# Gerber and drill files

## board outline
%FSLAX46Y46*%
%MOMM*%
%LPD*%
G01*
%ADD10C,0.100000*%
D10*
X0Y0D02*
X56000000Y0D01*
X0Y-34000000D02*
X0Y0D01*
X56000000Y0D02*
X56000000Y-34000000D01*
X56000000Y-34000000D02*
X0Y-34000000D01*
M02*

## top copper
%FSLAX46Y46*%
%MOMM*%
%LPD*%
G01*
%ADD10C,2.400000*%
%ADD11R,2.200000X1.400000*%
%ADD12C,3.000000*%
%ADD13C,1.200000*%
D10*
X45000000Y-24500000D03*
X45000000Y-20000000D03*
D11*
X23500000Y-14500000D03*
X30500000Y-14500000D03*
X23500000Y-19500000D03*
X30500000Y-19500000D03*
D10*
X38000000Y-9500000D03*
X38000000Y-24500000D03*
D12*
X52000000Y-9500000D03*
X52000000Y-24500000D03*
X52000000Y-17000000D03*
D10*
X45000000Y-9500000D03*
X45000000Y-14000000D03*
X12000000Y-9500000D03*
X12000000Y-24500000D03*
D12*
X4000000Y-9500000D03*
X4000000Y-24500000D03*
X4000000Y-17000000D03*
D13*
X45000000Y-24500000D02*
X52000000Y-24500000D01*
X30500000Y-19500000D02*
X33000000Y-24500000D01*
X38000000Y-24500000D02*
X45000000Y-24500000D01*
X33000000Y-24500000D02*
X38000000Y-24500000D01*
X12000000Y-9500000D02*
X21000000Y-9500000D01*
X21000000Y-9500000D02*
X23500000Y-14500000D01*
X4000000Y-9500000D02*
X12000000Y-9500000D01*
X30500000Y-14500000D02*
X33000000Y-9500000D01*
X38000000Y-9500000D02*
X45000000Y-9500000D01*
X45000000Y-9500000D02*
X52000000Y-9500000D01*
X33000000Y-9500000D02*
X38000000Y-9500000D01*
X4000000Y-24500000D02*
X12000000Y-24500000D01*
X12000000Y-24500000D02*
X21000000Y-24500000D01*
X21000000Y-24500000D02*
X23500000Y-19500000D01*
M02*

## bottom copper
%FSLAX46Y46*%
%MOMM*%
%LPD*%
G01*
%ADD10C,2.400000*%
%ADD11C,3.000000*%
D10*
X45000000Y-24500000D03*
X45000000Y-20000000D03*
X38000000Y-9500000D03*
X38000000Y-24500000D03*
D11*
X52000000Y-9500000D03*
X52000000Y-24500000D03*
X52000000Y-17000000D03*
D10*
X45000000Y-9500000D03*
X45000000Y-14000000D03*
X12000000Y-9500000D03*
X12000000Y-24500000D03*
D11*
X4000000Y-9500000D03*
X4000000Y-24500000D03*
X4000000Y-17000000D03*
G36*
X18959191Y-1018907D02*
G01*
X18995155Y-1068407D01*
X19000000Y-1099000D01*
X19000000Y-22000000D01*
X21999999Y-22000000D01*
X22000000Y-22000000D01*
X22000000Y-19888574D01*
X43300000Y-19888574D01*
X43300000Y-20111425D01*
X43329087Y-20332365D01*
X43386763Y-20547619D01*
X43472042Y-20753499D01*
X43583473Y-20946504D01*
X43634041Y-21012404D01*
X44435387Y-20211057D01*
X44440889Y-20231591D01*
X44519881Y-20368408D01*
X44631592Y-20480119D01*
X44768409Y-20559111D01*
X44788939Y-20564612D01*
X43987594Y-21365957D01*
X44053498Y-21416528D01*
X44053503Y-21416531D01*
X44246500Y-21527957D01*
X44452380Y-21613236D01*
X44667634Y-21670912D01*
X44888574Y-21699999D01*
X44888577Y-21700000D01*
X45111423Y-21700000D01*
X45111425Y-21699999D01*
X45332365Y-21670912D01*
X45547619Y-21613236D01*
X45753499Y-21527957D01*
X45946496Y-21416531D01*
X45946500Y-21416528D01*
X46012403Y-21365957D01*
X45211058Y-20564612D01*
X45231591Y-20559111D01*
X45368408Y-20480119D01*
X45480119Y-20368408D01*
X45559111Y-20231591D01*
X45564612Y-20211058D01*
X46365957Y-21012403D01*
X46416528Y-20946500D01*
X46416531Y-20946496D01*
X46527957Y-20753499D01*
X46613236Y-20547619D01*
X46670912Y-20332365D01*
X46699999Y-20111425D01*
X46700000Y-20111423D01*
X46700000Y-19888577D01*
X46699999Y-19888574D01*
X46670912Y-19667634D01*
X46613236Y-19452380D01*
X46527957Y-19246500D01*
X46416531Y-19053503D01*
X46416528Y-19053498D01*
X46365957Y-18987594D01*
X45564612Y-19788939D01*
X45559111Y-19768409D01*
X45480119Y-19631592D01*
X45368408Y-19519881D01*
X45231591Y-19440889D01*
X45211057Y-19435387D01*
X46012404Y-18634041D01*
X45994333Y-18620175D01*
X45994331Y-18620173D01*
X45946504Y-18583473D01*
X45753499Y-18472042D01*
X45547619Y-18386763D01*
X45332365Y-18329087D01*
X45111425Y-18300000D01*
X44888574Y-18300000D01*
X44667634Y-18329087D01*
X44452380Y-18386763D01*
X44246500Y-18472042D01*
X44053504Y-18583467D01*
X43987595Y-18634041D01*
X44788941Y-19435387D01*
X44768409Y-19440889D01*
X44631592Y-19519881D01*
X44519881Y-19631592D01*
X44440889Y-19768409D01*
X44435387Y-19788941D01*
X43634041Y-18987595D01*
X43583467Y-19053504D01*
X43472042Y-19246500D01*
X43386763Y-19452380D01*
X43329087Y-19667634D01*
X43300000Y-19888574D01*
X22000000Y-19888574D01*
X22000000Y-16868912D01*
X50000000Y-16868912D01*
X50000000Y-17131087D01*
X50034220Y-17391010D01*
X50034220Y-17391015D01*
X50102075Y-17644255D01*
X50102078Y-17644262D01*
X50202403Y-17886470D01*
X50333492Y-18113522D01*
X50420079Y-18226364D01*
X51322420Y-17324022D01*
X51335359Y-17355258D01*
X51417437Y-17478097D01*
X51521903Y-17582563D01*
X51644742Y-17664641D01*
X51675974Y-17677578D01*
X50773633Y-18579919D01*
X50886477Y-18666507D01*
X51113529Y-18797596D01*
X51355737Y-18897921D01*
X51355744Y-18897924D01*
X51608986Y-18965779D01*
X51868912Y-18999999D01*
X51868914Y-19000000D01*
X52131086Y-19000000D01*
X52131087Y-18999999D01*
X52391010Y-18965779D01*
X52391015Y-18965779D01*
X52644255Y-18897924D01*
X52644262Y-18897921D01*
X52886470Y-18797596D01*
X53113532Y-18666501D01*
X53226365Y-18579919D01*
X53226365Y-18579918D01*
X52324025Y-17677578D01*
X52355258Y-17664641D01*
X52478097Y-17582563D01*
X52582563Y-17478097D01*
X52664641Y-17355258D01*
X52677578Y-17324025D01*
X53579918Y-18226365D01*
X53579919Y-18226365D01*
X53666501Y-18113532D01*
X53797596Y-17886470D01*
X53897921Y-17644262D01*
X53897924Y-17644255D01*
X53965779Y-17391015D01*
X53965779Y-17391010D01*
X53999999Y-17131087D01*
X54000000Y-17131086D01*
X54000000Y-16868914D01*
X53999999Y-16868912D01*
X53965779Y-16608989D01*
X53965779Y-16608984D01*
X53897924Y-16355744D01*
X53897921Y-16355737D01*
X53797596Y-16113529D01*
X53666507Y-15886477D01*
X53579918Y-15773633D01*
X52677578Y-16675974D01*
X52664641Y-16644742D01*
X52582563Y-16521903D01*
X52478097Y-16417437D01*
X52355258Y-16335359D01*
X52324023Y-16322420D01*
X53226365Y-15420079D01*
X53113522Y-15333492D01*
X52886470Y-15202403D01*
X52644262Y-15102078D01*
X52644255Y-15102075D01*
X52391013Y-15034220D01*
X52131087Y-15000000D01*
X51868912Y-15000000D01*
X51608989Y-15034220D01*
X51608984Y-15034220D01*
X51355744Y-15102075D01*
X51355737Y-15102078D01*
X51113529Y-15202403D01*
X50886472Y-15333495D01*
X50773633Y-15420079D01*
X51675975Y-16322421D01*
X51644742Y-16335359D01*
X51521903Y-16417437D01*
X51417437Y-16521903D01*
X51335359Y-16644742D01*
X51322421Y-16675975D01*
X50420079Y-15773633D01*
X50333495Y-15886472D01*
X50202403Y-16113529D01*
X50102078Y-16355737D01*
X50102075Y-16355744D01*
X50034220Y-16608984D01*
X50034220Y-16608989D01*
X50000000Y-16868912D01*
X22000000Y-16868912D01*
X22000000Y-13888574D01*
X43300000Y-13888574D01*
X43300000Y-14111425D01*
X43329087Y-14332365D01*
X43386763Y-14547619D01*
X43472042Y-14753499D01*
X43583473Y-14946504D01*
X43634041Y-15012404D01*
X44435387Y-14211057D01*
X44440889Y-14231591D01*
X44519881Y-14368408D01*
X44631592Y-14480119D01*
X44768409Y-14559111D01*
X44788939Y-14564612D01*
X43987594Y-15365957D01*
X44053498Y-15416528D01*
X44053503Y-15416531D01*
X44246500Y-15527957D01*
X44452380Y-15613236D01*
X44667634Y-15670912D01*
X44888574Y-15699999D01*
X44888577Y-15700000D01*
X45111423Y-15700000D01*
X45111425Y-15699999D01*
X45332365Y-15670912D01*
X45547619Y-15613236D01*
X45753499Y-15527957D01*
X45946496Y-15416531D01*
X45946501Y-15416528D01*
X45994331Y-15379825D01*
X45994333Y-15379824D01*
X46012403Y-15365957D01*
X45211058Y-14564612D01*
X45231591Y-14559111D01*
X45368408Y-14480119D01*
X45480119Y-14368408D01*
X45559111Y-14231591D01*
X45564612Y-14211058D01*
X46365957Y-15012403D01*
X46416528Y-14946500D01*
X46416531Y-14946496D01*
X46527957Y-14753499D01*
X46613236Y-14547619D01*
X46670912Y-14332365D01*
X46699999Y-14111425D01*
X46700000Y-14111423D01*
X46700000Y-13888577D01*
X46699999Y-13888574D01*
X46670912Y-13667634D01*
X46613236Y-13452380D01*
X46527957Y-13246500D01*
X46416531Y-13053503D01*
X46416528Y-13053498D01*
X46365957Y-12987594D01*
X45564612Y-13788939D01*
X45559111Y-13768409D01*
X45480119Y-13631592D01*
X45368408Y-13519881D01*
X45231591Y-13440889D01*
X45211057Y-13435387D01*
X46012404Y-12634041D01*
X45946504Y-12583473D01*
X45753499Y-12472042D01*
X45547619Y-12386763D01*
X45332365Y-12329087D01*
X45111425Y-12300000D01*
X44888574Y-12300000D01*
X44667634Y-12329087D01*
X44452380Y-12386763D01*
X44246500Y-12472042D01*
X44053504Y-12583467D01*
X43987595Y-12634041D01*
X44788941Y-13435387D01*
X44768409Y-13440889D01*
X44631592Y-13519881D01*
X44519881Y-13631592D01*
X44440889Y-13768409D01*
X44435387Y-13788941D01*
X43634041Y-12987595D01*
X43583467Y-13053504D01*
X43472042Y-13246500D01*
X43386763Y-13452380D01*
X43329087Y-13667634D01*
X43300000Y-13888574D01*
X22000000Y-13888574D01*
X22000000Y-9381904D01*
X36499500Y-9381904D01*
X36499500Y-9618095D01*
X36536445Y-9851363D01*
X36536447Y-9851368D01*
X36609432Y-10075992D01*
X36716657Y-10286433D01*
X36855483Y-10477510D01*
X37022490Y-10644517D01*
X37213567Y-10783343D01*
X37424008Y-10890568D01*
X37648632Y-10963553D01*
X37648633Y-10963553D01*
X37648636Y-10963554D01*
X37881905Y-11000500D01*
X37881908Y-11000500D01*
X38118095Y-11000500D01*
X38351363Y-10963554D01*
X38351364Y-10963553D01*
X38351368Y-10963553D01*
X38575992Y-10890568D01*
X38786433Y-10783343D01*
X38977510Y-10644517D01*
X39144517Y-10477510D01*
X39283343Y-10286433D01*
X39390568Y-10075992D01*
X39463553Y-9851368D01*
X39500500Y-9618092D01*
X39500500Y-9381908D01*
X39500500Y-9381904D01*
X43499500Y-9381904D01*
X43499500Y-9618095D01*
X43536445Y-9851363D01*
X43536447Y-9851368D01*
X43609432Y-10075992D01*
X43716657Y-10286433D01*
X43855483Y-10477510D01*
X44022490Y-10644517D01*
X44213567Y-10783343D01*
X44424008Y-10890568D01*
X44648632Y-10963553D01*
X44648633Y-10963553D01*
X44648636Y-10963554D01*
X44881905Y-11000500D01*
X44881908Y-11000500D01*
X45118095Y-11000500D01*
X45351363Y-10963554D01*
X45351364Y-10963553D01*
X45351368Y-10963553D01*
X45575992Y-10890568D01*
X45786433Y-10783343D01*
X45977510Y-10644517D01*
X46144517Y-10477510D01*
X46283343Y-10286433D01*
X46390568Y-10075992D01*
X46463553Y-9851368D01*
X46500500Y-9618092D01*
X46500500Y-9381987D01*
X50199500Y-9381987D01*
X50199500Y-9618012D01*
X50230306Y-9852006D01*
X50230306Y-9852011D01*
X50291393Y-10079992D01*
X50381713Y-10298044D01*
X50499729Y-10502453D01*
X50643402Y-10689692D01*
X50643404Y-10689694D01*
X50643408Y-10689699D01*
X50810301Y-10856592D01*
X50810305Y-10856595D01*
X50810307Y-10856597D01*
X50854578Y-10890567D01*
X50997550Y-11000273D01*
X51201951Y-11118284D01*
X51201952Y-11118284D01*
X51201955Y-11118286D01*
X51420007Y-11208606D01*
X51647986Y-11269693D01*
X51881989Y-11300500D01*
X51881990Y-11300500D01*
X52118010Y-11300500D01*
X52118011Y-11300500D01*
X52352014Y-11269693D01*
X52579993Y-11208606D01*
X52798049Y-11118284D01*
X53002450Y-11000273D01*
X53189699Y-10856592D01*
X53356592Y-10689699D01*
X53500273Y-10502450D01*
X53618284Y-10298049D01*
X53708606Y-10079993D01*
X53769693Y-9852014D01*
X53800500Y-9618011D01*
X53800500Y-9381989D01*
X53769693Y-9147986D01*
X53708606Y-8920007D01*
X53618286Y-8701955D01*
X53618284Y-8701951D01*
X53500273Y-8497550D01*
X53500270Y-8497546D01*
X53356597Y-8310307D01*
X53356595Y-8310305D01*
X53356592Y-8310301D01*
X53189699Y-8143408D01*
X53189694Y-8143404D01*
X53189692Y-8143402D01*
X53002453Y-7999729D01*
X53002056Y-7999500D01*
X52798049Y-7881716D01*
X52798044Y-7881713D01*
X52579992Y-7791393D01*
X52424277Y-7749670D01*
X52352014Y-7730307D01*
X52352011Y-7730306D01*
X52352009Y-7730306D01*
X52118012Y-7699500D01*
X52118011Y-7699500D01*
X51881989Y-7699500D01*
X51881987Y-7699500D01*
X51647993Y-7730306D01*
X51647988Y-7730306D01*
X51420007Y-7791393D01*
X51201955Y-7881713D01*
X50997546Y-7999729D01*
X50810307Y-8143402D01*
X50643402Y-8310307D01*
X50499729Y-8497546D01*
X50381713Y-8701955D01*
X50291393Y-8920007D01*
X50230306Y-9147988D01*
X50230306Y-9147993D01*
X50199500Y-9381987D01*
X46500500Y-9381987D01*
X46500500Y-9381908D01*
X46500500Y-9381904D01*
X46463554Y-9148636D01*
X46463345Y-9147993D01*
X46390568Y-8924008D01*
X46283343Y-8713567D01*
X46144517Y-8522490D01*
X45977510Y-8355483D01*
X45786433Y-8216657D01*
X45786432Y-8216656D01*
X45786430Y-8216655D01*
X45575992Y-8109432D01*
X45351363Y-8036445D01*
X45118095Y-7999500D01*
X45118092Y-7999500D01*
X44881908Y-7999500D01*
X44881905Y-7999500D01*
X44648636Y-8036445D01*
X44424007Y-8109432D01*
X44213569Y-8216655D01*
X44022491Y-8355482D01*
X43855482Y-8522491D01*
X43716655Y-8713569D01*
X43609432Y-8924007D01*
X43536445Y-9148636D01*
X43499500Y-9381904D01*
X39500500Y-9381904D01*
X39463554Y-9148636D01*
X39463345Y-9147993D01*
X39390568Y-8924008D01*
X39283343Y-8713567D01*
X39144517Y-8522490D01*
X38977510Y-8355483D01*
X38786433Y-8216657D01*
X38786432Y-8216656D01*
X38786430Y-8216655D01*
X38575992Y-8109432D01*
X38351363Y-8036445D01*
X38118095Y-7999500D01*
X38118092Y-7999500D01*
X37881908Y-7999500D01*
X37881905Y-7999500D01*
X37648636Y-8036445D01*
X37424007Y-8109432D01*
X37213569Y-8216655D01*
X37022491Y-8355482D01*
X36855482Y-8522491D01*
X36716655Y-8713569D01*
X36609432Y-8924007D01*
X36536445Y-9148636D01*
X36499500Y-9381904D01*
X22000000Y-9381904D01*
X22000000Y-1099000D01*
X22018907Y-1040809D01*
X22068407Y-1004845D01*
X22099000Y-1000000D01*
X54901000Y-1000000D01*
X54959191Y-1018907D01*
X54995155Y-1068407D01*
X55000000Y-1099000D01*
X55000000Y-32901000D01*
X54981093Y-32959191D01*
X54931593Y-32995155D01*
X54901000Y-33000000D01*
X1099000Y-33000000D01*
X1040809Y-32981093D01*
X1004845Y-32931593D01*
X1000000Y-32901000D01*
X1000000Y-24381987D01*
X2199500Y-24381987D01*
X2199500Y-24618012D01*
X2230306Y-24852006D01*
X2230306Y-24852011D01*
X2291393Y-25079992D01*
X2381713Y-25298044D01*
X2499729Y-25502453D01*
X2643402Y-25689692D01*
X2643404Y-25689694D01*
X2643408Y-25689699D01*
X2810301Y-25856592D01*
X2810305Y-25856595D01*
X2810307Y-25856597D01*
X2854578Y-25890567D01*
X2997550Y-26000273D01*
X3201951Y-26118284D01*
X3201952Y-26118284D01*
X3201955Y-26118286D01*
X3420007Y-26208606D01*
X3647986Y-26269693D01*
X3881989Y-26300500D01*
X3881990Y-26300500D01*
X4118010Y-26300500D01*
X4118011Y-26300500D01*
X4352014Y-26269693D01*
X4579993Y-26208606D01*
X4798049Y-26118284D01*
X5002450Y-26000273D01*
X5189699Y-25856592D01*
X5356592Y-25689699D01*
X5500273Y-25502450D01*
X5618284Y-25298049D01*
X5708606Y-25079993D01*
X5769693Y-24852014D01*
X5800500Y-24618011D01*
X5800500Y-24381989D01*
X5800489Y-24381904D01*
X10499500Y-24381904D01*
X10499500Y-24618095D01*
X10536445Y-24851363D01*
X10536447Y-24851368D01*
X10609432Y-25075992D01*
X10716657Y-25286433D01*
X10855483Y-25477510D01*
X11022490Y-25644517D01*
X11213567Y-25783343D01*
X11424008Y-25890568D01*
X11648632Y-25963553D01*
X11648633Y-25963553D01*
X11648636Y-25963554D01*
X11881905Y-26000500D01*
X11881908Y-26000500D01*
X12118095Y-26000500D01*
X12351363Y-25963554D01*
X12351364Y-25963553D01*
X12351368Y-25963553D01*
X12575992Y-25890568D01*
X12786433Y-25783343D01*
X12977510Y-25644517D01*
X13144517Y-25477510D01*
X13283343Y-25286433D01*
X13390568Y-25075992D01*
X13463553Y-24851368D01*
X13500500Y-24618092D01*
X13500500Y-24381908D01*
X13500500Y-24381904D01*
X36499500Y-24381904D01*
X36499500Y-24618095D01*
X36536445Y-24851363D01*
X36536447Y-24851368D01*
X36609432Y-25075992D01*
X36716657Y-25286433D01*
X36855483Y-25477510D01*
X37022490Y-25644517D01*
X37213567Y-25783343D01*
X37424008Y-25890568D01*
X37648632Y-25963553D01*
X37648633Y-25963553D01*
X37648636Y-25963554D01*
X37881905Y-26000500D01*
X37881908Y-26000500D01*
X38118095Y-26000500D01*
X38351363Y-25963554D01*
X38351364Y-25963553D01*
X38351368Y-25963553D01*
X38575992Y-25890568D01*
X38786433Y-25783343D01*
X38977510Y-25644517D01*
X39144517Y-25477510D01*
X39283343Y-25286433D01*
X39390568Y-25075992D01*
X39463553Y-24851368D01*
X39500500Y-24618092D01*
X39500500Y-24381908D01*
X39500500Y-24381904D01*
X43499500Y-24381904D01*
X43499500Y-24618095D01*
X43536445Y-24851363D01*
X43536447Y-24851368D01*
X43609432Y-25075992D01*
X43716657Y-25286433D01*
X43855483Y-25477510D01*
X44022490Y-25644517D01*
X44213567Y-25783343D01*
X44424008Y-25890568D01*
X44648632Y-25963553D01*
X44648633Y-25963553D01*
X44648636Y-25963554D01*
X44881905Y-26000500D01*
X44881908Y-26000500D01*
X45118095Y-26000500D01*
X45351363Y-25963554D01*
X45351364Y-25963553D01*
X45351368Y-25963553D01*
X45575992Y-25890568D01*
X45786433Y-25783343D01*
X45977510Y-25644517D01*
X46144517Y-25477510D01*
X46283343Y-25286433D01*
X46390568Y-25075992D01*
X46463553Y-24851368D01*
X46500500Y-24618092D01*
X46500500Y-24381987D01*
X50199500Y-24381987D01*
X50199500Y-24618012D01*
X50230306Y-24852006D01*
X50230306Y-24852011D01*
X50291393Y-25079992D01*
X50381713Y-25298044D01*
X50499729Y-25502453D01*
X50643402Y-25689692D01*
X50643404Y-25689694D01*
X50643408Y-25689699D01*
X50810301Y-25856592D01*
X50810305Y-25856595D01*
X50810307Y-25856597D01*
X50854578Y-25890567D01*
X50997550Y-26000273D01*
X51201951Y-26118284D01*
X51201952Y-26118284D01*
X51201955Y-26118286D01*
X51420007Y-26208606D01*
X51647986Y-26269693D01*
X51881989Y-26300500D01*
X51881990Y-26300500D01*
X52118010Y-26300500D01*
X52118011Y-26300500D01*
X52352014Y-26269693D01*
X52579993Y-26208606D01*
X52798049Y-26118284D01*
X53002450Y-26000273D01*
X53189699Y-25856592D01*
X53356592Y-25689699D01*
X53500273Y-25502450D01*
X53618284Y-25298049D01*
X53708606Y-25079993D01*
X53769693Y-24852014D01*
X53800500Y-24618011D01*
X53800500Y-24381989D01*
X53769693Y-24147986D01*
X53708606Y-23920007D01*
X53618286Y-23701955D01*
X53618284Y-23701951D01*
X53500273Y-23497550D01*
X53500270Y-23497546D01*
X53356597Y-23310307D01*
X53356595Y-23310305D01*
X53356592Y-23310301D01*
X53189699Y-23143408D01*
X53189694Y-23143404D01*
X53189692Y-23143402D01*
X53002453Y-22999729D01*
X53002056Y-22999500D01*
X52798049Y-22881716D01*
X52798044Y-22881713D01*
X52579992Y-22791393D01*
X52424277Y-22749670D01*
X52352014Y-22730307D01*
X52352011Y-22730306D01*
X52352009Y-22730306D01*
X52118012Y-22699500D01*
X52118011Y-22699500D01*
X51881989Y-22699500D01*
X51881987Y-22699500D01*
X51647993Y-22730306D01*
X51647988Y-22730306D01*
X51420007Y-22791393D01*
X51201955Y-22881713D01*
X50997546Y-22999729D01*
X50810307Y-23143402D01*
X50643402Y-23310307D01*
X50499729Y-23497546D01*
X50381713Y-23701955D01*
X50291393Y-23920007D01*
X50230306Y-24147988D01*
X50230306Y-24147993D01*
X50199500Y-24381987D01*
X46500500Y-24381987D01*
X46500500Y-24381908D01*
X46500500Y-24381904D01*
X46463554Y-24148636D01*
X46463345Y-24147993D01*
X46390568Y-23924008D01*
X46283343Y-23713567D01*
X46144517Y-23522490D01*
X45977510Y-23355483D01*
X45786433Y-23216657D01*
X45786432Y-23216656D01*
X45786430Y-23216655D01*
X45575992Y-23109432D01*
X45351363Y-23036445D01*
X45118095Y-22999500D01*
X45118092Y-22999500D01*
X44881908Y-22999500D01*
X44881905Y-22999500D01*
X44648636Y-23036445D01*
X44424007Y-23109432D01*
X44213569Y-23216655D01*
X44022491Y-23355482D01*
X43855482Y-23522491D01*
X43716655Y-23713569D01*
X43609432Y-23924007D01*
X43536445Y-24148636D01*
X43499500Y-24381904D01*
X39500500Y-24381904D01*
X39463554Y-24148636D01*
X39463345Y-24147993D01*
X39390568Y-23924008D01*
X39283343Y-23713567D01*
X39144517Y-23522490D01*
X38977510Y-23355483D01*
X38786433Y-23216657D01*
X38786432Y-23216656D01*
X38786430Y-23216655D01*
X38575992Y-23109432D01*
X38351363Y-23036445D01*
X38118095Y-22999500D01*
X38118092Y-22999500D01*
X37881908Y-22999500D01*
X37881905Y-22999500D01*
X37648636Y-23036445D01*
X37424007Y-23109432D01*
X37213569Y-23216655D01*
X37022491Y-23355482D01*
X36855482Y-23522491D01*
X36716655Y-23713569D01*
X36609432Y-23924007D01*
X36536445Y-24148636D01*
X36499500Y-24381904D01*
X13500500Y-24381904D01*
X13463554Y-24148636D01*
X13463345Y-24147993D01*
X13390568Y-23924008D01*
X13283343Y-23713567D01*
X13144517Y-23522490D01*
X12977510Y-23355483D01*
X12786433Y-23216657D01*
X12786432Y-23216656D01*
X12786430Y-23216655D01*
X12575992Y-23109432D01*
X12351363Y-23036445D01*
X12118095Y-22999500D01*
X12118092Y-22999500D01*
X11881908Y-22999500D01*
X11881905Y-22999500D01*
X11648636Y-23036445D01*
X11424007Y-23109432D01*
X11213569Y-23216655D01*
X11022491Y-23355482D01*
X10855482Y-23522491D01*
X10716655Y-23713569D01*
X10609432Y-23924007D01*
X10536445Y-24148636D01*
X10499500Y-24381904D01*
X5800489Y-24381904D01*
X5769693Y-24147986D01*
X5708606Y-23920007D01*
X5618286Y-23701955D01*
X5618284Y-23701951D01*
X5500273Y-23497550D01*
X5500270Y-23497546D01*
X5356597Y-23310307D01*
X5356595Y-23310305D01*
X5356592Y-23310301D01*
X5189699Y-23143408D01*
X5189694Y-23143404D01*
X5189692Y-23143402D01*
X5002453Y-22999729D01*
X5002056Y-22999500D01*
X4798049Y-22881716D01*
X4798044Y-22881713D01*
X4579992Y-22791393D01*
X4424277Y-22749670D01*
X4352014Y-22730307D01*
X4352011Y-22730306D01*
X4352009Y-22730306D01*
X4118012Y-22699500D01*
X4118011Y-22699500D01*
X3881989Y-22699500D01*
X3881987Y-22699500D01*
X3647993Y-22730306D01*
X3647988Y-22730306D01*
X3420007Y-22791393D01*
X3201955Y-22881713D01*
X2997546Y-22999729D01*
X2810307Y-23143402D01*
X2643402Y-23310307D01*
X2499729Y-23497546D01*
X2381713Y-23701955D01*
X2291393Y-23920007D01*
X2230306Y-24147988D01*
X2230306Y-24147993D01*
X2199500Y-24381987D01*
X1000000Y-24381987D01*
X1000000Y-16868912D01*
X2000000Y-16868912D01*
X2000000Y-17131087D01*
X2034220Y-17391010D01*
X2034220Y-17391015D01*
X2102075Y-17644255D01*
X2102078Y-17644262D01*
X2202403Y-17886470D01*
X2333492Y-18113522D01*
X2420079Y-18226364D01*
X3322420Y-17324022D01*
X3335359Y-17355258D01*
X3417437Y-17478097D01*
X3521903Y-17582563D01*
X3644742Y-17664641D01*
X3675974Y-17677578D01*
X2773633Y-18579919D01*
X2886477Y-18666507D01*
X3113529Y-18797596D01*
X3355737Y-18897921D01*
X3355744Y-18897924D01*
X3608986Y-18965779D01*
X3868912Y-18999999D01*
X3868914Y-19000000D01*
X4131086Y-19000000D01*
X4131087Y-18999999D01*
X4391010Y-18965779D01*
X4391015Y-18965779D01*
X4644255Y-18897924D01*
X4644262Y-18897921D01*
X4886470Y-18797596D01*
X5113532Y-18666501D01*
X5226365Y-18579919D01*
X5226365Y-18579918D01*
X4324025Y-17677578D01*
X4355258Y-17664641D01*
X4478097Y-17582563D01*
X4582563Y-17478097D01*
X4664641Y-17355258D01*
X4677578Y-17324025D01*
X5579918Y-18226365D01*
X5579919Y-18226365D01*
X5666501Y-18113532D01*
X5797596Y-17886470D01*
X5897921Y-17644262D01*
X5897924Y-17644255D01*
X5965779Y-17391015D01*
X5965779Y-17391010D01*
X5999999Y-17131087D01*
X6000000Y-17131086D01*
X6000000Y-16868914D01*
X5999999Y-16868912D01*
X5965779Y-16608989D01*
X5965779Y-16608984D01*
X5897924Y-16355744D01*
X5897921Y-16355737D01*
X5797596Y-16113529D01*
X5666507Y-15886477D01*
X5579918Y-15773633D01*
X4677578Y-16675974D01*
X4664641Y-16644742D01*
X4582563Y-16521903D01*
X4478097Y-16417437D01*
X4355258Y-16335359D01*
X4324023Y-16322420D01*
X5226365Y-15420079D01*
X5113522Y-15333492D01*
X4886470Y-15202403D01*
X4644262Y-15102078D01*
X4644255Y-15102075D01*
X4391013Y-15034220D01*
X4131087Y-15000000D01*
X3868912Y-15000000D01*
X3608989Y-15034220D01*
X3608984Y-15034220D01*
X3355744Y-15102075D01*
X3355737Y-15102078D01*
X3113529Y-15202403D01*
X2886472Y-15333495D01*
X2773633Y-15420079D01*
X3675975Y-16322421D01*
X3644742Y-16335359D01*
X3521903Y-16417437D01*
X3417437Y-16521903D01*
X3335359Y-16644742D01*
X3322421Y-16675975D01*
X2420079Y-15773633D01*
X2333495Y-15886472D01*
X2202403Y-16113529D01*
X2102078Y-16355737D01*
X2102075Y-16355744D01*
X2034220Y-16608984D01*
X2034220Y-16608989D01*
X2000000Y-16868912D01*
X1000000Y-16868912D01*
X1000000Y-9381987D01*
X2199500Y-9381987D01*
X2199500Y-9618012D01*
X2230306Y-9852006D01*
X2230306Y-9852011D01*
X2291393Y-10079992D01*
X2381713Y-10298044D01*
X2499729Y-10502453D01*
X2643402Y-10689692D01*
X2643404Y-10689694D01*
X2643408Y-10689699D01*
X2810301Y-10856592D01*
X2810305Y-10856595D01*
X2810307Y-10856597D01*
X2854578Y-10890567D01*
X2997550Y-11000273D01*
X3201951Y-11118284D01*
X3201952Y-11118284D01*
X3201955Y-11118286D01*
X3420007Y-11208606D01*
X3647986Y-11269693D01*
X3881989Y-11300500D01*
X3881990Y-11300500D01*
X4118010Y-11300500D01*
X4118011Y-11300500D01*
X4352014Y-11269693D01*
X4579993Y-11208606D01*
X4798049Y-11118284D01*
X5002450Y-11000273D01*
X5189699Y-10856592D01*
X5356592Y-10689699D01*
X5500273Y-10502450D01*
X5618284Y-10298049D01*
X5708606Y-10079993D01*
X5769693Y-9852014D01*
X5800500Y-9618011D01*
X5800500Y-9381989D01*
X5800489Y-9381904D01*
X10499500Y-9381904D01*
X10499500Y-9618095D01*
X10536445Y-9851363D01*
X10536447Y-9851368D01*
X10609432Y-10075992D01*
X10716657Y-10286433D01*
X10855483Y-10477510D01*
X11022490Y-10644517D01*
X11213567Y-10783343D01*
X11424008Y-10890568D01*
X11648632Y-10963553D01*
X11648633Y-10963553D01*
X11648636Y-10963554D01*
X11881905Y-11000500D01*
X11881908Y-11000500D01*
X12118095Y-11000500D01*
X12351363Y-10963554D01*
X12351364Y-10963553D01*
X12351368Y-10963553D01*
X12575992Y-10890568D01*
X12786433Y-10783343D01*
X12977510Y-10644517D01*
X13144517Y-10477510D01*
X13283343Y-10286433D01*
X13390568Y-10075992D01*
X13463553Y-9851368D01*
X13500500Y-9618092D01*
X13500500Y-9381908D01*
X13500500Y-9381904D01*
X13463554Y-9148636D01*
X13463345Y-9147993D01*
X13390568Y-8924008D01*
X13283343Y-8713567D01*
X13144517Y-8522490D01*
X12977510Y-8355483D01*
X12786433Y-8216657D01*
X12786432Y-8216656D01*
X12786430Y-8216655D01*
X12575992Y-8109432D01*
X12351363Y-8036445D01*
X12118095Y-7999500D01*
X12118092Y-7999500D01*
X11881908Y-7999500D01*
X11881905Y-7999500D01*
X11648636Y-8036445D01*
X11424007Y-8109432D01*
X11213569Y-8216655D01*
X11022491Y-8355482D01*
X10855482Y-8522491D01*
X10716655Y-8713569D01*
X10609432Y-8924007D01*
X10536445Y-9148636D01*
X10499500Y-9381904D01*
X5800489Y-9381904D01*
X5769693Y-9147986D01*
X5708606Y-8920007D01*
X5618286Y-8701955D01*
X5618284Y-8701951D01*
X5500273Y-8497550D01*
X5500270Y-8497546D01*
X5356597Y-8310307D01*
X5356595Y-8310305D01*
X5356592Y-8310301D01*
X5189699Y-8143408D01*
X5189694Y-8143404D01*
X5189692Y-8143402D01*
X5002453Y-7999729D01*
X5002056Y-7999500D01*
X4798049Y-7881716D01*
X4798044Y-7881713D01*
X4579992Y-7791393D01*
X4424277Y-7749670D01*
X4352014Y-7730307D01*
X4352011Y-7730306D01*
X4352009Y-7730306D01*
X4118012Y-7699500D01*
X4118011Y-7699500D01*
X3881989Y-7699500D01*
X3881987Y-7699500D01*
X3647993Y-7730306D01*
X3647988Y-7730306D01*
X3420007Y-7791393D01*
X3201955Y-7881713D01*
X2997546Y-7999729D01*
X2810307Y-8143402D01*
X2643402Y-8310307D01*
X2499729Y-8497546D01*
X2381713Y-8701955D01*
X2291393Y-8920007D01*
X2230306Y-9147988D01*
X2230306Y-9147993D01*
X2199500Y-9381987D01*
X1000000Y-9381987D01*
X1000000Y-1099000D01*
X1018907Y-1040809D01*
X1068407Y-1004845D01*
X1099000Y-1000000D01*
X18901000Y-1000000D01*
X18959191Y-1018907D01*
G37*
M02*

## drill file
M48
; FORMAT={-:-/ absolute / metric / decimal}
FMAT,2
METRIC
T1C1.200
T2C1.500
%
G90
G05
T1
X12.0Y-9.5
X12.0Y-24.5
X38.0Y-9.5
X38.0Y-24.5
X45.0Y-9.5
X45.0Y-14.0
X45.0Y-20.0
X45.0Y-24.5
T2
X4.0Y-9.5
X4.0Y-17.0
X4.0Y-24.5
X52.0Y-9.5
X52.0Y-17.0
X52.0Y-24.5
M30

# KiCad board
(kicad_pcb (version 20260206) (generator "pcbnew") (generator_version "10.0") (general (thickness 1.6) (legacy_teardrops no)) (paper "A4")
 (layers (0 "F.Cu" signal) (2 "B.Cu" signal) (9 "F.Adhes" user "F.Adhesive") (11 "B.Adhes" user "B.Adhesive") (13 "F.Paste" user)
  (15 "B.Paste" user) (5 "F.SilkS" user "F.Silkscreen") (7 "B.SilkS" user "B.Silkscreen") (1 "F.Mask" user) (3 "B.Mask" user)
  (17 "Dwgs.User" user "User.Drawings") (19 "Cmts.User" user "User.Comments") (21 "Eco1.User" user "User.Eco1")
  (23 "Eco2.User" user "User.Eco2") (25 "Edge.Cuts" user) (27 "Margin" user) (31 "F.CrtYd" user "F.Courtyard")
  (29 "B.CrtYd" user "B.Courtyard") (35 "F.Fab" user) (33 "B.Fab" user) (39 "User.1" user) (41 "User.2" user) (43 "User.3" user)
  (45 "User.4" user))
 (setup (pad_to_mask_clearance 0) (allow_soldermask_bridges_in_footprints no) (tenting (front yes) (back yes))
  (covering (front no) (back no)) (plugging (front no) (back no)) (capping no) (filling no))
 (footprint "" (layer "F.Cu") (at 0 0)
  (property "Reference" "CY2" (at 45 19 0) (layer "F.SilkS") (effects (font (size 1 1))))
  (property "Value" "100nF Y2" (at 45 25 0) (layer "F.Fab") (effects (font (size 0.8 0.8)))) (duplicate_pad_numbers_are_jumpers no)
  (pad "1" thru_hole circle (at 45 24.5) (size 2.4 2.4) (drill 1.2) (layers "*.Cu" "*.Mask") (remove_unused_layers no) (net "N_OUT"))
  (pad "2" thru_hole circle (at 45 20) (size 2.4 2.4) (drill 1.2) (layers "*.Cu" "*.Mask") (remove_unused_layers no) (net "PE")))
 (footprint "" (layer "F.Cu") (at 0 0)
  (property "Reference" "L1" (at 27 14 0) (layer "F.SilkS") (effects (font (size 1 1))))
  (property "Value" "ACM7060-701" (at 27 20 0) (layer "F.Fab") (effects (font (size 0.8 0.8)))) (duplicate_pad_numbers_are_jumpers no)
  (pad "1" smd rect (at 23.5 14.5) (size 2.2 1.4) (layers "F.Cu" "F.Mask" "F.Paste") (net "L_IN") (thermal_bridge_angle 45))
  (pad "2" smd rect (at 30.5 14.5) (size 2.2 1.4) (layers "F.Cu" "F.Mask" "F.Paste") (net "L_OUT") (thermal_bridge_angle 45))
  (pad "3" smd rect (at 23.5 19.5) (size 2.2 1.4) (layers "F.Cu" "F.Mask" "F.Paste") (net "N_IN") (thermal_bridge_angle 45))
  (pad "4" smd rect (at 30.5 19.5) (size 2.2 1.4) (layers "F.Cu" "F.Mask" "F.Paste") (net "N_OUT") (thermal_bridge_angle 45)))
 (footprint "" (layer "F.Cu") (at 0 0)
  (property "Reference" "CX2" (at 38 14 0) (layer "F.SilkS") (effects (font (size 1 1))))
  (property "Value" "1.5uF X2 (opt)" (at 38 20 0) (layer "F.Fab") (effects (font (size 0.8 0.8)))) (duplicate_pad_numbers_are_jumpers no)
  (pad "1" thru_hole circle (at 38 9.5) (size 2.4 2.4) (drill 1.2) (layers "*.Cu" "*.Mask") (remove_unused_layers no) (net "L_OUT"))
  (pad "2" thru_hole circle (at 38 24.5) (size 2.4 2.4) (drill 1.2) (layers "*.Cu" "*.Mask") (remove_unused_layers no) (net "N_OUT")))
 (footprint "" (layer "F.Cu") (at 0 0)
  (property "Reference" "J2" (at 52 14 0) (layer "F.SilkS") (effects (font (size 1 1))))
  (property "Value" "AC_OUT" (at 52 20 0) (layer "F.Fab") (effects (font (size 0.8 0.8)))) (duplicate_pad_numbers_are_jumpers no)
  (pad "1" thru_hole circle (at 52 9.5) (size 3 3) (drill 1.5) (layers "*.Cu" "*.Mask") (remove_unused_layers no) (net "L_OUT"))
  (pad "2" thru_hole circle (at 52 24.5) (size 3 3) (drill 1.5) (layers "*.Cu" "*.Mask") (remove_unused_layers no) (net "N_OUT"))
  (pad "3" thru_hole circle (at 52 17) (size 3 3) (drill 1.5) (layers "*.Cu" "*.Mask") (remove_unused_layers no) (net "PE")))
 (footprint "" (layer "F.Cu") (at 0 0)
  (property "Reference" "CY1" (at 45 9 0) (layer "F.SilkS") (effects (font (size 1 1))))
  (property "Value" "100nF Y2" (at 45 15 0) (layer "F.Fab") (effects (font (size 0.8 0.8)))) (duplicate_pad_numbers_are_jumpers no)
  (pad "1" thru_hole circle (at 45 9.5) (size 2.4 2.4) (drill 1.2) (layers "*.Cu" "*.Mask") (remove_unused_layers no) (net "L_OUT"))
  (pad "2" thru_hole circle (at 45 14) (size 2.4 2.4) (drill 1.2) (layers "*.Cu" "*.Mask") (remove_unused_layers no) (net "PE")))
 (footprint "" (layer "F.Cu") (at 0 0)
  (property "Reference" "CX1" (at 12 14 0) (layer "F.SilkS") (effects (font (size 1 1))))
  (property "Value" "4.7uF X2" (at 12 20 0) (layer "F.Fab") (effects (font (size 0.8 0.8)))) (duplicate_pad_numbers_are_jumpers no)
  (pad "1" thru_hole circle (at 12 9.5) (size 2.4 2.4) (drill 1.2) (layers "*.Cu" "*.Mask") (remove_unused_layers no) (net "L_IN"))
  (pad "2" thru_hole circle (at 12 24.5) (size 2.4 2.4) (drill 1.2) (layers "*.Cu" "*.Mask") (remove_unused_layers no) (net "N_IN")))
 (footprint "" (layer "F.Cu") (at 0 0)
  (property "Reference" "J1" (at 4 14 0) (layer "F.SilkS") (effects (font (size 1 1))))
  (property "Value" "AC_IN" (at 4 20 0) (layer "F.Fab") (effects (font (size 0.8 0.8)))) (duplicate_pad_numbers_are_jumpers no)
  (pad "1" thru_hole circle (at 4 9.5) (size 3 3) (drill 1.5) (layers "*.Cu" "*.Mask") (remove_unused_layers no) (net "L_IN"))
  (pad "2" thru_hole circle (at 4 24.5) (size 3 3) (drill 1.5) (layers "*.Cu" "*.Mask") (remove_unused_layers no) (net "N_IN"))
  (pad "3" thru_hole circle (at 4 17) (size 3 3) (drill 1.5) (layers "*.Cu" "*.Mask") (remove_unused_layers no) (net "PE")))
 (gr_line (start 0 0) (end 56 0) (stroke (width 0.1) (type default)) (layer "Edge.Cuts"))
 (gr_line (start 0 34) (end 0 0) (stroke (width 0.1) (type default)) (layer "Edge.Cuts"))
 (gr_line (start 56 0) (end 56 34) (stroke (width 0.1) (type default)) (layer "Edge.Cuts"))
 (gr_line (start 56 34) (end 0 34) (stroke (width 0.1) (type default)) (layer "Edge.Cuts"))
 (segment (start 45 24.5) (end 52 24.5) (width 1.2) (layer "F.Cu") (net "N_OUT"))
 (segment (start 30.5 19.5) (end 33 24.5) (width 1.2) (layer "F.Cu") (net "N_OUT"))
 (segment (start 38 24.5) (end 45 24.5) (width 1.2) (layer "F.Cu") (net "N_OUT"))
 (segment (start 33 24.5) (end 38 24.5) (width 1.2) (layer "F.Cu") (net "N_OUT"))
 (segment (start 12 9.5) (end 21 9.5) (width 1.2) (layer "F.Cu") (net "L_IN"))
 (segment (start 21 9.5) (end 23.5 14.5) (width 1.2) (layer "F.Cu") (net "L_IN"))
 (segment (start 4 9.5) (end 12 9.5) (width 1.2) (layer "F.Cu") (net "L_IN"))
 (segment (start 30.5 14.5) (end 33 9.5) (width 1.2) (layer "F.Cu") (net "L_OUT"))
 (segment (start 38 9.5) (end 45 9.5) (width 1.2) (layer "F.Cu") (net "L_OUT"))
 (segment (start 45 9.5) (end 52 9.5) (width 1.2) (layer "F.Cu") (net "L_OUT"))
 (segment (start 33 9.5) (end 38 9.5) (width 1.2) (layer "F.Cu") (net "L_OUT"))
 (segment (start 4 24.5) (end 12 24.5) (width 1.2) (layer "F.Cu") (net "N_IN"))
 (segment (start 12 24.5) (end 21 24.5) (width 1.2) (layer "F.Cu") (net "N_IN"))
 (segment (start 21 24.5) (end 23.5 19.5) (width 1.2) (layer "F.Cu") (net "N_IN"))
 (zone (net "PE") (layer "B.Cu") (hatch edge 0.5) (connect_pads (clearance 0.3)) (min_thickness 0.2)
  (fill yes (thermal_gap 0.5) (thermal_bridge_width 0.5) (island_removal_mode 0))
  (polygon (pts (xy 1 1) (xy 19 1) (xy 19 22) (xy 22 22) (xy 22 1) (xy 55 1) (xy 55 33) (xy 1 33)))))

